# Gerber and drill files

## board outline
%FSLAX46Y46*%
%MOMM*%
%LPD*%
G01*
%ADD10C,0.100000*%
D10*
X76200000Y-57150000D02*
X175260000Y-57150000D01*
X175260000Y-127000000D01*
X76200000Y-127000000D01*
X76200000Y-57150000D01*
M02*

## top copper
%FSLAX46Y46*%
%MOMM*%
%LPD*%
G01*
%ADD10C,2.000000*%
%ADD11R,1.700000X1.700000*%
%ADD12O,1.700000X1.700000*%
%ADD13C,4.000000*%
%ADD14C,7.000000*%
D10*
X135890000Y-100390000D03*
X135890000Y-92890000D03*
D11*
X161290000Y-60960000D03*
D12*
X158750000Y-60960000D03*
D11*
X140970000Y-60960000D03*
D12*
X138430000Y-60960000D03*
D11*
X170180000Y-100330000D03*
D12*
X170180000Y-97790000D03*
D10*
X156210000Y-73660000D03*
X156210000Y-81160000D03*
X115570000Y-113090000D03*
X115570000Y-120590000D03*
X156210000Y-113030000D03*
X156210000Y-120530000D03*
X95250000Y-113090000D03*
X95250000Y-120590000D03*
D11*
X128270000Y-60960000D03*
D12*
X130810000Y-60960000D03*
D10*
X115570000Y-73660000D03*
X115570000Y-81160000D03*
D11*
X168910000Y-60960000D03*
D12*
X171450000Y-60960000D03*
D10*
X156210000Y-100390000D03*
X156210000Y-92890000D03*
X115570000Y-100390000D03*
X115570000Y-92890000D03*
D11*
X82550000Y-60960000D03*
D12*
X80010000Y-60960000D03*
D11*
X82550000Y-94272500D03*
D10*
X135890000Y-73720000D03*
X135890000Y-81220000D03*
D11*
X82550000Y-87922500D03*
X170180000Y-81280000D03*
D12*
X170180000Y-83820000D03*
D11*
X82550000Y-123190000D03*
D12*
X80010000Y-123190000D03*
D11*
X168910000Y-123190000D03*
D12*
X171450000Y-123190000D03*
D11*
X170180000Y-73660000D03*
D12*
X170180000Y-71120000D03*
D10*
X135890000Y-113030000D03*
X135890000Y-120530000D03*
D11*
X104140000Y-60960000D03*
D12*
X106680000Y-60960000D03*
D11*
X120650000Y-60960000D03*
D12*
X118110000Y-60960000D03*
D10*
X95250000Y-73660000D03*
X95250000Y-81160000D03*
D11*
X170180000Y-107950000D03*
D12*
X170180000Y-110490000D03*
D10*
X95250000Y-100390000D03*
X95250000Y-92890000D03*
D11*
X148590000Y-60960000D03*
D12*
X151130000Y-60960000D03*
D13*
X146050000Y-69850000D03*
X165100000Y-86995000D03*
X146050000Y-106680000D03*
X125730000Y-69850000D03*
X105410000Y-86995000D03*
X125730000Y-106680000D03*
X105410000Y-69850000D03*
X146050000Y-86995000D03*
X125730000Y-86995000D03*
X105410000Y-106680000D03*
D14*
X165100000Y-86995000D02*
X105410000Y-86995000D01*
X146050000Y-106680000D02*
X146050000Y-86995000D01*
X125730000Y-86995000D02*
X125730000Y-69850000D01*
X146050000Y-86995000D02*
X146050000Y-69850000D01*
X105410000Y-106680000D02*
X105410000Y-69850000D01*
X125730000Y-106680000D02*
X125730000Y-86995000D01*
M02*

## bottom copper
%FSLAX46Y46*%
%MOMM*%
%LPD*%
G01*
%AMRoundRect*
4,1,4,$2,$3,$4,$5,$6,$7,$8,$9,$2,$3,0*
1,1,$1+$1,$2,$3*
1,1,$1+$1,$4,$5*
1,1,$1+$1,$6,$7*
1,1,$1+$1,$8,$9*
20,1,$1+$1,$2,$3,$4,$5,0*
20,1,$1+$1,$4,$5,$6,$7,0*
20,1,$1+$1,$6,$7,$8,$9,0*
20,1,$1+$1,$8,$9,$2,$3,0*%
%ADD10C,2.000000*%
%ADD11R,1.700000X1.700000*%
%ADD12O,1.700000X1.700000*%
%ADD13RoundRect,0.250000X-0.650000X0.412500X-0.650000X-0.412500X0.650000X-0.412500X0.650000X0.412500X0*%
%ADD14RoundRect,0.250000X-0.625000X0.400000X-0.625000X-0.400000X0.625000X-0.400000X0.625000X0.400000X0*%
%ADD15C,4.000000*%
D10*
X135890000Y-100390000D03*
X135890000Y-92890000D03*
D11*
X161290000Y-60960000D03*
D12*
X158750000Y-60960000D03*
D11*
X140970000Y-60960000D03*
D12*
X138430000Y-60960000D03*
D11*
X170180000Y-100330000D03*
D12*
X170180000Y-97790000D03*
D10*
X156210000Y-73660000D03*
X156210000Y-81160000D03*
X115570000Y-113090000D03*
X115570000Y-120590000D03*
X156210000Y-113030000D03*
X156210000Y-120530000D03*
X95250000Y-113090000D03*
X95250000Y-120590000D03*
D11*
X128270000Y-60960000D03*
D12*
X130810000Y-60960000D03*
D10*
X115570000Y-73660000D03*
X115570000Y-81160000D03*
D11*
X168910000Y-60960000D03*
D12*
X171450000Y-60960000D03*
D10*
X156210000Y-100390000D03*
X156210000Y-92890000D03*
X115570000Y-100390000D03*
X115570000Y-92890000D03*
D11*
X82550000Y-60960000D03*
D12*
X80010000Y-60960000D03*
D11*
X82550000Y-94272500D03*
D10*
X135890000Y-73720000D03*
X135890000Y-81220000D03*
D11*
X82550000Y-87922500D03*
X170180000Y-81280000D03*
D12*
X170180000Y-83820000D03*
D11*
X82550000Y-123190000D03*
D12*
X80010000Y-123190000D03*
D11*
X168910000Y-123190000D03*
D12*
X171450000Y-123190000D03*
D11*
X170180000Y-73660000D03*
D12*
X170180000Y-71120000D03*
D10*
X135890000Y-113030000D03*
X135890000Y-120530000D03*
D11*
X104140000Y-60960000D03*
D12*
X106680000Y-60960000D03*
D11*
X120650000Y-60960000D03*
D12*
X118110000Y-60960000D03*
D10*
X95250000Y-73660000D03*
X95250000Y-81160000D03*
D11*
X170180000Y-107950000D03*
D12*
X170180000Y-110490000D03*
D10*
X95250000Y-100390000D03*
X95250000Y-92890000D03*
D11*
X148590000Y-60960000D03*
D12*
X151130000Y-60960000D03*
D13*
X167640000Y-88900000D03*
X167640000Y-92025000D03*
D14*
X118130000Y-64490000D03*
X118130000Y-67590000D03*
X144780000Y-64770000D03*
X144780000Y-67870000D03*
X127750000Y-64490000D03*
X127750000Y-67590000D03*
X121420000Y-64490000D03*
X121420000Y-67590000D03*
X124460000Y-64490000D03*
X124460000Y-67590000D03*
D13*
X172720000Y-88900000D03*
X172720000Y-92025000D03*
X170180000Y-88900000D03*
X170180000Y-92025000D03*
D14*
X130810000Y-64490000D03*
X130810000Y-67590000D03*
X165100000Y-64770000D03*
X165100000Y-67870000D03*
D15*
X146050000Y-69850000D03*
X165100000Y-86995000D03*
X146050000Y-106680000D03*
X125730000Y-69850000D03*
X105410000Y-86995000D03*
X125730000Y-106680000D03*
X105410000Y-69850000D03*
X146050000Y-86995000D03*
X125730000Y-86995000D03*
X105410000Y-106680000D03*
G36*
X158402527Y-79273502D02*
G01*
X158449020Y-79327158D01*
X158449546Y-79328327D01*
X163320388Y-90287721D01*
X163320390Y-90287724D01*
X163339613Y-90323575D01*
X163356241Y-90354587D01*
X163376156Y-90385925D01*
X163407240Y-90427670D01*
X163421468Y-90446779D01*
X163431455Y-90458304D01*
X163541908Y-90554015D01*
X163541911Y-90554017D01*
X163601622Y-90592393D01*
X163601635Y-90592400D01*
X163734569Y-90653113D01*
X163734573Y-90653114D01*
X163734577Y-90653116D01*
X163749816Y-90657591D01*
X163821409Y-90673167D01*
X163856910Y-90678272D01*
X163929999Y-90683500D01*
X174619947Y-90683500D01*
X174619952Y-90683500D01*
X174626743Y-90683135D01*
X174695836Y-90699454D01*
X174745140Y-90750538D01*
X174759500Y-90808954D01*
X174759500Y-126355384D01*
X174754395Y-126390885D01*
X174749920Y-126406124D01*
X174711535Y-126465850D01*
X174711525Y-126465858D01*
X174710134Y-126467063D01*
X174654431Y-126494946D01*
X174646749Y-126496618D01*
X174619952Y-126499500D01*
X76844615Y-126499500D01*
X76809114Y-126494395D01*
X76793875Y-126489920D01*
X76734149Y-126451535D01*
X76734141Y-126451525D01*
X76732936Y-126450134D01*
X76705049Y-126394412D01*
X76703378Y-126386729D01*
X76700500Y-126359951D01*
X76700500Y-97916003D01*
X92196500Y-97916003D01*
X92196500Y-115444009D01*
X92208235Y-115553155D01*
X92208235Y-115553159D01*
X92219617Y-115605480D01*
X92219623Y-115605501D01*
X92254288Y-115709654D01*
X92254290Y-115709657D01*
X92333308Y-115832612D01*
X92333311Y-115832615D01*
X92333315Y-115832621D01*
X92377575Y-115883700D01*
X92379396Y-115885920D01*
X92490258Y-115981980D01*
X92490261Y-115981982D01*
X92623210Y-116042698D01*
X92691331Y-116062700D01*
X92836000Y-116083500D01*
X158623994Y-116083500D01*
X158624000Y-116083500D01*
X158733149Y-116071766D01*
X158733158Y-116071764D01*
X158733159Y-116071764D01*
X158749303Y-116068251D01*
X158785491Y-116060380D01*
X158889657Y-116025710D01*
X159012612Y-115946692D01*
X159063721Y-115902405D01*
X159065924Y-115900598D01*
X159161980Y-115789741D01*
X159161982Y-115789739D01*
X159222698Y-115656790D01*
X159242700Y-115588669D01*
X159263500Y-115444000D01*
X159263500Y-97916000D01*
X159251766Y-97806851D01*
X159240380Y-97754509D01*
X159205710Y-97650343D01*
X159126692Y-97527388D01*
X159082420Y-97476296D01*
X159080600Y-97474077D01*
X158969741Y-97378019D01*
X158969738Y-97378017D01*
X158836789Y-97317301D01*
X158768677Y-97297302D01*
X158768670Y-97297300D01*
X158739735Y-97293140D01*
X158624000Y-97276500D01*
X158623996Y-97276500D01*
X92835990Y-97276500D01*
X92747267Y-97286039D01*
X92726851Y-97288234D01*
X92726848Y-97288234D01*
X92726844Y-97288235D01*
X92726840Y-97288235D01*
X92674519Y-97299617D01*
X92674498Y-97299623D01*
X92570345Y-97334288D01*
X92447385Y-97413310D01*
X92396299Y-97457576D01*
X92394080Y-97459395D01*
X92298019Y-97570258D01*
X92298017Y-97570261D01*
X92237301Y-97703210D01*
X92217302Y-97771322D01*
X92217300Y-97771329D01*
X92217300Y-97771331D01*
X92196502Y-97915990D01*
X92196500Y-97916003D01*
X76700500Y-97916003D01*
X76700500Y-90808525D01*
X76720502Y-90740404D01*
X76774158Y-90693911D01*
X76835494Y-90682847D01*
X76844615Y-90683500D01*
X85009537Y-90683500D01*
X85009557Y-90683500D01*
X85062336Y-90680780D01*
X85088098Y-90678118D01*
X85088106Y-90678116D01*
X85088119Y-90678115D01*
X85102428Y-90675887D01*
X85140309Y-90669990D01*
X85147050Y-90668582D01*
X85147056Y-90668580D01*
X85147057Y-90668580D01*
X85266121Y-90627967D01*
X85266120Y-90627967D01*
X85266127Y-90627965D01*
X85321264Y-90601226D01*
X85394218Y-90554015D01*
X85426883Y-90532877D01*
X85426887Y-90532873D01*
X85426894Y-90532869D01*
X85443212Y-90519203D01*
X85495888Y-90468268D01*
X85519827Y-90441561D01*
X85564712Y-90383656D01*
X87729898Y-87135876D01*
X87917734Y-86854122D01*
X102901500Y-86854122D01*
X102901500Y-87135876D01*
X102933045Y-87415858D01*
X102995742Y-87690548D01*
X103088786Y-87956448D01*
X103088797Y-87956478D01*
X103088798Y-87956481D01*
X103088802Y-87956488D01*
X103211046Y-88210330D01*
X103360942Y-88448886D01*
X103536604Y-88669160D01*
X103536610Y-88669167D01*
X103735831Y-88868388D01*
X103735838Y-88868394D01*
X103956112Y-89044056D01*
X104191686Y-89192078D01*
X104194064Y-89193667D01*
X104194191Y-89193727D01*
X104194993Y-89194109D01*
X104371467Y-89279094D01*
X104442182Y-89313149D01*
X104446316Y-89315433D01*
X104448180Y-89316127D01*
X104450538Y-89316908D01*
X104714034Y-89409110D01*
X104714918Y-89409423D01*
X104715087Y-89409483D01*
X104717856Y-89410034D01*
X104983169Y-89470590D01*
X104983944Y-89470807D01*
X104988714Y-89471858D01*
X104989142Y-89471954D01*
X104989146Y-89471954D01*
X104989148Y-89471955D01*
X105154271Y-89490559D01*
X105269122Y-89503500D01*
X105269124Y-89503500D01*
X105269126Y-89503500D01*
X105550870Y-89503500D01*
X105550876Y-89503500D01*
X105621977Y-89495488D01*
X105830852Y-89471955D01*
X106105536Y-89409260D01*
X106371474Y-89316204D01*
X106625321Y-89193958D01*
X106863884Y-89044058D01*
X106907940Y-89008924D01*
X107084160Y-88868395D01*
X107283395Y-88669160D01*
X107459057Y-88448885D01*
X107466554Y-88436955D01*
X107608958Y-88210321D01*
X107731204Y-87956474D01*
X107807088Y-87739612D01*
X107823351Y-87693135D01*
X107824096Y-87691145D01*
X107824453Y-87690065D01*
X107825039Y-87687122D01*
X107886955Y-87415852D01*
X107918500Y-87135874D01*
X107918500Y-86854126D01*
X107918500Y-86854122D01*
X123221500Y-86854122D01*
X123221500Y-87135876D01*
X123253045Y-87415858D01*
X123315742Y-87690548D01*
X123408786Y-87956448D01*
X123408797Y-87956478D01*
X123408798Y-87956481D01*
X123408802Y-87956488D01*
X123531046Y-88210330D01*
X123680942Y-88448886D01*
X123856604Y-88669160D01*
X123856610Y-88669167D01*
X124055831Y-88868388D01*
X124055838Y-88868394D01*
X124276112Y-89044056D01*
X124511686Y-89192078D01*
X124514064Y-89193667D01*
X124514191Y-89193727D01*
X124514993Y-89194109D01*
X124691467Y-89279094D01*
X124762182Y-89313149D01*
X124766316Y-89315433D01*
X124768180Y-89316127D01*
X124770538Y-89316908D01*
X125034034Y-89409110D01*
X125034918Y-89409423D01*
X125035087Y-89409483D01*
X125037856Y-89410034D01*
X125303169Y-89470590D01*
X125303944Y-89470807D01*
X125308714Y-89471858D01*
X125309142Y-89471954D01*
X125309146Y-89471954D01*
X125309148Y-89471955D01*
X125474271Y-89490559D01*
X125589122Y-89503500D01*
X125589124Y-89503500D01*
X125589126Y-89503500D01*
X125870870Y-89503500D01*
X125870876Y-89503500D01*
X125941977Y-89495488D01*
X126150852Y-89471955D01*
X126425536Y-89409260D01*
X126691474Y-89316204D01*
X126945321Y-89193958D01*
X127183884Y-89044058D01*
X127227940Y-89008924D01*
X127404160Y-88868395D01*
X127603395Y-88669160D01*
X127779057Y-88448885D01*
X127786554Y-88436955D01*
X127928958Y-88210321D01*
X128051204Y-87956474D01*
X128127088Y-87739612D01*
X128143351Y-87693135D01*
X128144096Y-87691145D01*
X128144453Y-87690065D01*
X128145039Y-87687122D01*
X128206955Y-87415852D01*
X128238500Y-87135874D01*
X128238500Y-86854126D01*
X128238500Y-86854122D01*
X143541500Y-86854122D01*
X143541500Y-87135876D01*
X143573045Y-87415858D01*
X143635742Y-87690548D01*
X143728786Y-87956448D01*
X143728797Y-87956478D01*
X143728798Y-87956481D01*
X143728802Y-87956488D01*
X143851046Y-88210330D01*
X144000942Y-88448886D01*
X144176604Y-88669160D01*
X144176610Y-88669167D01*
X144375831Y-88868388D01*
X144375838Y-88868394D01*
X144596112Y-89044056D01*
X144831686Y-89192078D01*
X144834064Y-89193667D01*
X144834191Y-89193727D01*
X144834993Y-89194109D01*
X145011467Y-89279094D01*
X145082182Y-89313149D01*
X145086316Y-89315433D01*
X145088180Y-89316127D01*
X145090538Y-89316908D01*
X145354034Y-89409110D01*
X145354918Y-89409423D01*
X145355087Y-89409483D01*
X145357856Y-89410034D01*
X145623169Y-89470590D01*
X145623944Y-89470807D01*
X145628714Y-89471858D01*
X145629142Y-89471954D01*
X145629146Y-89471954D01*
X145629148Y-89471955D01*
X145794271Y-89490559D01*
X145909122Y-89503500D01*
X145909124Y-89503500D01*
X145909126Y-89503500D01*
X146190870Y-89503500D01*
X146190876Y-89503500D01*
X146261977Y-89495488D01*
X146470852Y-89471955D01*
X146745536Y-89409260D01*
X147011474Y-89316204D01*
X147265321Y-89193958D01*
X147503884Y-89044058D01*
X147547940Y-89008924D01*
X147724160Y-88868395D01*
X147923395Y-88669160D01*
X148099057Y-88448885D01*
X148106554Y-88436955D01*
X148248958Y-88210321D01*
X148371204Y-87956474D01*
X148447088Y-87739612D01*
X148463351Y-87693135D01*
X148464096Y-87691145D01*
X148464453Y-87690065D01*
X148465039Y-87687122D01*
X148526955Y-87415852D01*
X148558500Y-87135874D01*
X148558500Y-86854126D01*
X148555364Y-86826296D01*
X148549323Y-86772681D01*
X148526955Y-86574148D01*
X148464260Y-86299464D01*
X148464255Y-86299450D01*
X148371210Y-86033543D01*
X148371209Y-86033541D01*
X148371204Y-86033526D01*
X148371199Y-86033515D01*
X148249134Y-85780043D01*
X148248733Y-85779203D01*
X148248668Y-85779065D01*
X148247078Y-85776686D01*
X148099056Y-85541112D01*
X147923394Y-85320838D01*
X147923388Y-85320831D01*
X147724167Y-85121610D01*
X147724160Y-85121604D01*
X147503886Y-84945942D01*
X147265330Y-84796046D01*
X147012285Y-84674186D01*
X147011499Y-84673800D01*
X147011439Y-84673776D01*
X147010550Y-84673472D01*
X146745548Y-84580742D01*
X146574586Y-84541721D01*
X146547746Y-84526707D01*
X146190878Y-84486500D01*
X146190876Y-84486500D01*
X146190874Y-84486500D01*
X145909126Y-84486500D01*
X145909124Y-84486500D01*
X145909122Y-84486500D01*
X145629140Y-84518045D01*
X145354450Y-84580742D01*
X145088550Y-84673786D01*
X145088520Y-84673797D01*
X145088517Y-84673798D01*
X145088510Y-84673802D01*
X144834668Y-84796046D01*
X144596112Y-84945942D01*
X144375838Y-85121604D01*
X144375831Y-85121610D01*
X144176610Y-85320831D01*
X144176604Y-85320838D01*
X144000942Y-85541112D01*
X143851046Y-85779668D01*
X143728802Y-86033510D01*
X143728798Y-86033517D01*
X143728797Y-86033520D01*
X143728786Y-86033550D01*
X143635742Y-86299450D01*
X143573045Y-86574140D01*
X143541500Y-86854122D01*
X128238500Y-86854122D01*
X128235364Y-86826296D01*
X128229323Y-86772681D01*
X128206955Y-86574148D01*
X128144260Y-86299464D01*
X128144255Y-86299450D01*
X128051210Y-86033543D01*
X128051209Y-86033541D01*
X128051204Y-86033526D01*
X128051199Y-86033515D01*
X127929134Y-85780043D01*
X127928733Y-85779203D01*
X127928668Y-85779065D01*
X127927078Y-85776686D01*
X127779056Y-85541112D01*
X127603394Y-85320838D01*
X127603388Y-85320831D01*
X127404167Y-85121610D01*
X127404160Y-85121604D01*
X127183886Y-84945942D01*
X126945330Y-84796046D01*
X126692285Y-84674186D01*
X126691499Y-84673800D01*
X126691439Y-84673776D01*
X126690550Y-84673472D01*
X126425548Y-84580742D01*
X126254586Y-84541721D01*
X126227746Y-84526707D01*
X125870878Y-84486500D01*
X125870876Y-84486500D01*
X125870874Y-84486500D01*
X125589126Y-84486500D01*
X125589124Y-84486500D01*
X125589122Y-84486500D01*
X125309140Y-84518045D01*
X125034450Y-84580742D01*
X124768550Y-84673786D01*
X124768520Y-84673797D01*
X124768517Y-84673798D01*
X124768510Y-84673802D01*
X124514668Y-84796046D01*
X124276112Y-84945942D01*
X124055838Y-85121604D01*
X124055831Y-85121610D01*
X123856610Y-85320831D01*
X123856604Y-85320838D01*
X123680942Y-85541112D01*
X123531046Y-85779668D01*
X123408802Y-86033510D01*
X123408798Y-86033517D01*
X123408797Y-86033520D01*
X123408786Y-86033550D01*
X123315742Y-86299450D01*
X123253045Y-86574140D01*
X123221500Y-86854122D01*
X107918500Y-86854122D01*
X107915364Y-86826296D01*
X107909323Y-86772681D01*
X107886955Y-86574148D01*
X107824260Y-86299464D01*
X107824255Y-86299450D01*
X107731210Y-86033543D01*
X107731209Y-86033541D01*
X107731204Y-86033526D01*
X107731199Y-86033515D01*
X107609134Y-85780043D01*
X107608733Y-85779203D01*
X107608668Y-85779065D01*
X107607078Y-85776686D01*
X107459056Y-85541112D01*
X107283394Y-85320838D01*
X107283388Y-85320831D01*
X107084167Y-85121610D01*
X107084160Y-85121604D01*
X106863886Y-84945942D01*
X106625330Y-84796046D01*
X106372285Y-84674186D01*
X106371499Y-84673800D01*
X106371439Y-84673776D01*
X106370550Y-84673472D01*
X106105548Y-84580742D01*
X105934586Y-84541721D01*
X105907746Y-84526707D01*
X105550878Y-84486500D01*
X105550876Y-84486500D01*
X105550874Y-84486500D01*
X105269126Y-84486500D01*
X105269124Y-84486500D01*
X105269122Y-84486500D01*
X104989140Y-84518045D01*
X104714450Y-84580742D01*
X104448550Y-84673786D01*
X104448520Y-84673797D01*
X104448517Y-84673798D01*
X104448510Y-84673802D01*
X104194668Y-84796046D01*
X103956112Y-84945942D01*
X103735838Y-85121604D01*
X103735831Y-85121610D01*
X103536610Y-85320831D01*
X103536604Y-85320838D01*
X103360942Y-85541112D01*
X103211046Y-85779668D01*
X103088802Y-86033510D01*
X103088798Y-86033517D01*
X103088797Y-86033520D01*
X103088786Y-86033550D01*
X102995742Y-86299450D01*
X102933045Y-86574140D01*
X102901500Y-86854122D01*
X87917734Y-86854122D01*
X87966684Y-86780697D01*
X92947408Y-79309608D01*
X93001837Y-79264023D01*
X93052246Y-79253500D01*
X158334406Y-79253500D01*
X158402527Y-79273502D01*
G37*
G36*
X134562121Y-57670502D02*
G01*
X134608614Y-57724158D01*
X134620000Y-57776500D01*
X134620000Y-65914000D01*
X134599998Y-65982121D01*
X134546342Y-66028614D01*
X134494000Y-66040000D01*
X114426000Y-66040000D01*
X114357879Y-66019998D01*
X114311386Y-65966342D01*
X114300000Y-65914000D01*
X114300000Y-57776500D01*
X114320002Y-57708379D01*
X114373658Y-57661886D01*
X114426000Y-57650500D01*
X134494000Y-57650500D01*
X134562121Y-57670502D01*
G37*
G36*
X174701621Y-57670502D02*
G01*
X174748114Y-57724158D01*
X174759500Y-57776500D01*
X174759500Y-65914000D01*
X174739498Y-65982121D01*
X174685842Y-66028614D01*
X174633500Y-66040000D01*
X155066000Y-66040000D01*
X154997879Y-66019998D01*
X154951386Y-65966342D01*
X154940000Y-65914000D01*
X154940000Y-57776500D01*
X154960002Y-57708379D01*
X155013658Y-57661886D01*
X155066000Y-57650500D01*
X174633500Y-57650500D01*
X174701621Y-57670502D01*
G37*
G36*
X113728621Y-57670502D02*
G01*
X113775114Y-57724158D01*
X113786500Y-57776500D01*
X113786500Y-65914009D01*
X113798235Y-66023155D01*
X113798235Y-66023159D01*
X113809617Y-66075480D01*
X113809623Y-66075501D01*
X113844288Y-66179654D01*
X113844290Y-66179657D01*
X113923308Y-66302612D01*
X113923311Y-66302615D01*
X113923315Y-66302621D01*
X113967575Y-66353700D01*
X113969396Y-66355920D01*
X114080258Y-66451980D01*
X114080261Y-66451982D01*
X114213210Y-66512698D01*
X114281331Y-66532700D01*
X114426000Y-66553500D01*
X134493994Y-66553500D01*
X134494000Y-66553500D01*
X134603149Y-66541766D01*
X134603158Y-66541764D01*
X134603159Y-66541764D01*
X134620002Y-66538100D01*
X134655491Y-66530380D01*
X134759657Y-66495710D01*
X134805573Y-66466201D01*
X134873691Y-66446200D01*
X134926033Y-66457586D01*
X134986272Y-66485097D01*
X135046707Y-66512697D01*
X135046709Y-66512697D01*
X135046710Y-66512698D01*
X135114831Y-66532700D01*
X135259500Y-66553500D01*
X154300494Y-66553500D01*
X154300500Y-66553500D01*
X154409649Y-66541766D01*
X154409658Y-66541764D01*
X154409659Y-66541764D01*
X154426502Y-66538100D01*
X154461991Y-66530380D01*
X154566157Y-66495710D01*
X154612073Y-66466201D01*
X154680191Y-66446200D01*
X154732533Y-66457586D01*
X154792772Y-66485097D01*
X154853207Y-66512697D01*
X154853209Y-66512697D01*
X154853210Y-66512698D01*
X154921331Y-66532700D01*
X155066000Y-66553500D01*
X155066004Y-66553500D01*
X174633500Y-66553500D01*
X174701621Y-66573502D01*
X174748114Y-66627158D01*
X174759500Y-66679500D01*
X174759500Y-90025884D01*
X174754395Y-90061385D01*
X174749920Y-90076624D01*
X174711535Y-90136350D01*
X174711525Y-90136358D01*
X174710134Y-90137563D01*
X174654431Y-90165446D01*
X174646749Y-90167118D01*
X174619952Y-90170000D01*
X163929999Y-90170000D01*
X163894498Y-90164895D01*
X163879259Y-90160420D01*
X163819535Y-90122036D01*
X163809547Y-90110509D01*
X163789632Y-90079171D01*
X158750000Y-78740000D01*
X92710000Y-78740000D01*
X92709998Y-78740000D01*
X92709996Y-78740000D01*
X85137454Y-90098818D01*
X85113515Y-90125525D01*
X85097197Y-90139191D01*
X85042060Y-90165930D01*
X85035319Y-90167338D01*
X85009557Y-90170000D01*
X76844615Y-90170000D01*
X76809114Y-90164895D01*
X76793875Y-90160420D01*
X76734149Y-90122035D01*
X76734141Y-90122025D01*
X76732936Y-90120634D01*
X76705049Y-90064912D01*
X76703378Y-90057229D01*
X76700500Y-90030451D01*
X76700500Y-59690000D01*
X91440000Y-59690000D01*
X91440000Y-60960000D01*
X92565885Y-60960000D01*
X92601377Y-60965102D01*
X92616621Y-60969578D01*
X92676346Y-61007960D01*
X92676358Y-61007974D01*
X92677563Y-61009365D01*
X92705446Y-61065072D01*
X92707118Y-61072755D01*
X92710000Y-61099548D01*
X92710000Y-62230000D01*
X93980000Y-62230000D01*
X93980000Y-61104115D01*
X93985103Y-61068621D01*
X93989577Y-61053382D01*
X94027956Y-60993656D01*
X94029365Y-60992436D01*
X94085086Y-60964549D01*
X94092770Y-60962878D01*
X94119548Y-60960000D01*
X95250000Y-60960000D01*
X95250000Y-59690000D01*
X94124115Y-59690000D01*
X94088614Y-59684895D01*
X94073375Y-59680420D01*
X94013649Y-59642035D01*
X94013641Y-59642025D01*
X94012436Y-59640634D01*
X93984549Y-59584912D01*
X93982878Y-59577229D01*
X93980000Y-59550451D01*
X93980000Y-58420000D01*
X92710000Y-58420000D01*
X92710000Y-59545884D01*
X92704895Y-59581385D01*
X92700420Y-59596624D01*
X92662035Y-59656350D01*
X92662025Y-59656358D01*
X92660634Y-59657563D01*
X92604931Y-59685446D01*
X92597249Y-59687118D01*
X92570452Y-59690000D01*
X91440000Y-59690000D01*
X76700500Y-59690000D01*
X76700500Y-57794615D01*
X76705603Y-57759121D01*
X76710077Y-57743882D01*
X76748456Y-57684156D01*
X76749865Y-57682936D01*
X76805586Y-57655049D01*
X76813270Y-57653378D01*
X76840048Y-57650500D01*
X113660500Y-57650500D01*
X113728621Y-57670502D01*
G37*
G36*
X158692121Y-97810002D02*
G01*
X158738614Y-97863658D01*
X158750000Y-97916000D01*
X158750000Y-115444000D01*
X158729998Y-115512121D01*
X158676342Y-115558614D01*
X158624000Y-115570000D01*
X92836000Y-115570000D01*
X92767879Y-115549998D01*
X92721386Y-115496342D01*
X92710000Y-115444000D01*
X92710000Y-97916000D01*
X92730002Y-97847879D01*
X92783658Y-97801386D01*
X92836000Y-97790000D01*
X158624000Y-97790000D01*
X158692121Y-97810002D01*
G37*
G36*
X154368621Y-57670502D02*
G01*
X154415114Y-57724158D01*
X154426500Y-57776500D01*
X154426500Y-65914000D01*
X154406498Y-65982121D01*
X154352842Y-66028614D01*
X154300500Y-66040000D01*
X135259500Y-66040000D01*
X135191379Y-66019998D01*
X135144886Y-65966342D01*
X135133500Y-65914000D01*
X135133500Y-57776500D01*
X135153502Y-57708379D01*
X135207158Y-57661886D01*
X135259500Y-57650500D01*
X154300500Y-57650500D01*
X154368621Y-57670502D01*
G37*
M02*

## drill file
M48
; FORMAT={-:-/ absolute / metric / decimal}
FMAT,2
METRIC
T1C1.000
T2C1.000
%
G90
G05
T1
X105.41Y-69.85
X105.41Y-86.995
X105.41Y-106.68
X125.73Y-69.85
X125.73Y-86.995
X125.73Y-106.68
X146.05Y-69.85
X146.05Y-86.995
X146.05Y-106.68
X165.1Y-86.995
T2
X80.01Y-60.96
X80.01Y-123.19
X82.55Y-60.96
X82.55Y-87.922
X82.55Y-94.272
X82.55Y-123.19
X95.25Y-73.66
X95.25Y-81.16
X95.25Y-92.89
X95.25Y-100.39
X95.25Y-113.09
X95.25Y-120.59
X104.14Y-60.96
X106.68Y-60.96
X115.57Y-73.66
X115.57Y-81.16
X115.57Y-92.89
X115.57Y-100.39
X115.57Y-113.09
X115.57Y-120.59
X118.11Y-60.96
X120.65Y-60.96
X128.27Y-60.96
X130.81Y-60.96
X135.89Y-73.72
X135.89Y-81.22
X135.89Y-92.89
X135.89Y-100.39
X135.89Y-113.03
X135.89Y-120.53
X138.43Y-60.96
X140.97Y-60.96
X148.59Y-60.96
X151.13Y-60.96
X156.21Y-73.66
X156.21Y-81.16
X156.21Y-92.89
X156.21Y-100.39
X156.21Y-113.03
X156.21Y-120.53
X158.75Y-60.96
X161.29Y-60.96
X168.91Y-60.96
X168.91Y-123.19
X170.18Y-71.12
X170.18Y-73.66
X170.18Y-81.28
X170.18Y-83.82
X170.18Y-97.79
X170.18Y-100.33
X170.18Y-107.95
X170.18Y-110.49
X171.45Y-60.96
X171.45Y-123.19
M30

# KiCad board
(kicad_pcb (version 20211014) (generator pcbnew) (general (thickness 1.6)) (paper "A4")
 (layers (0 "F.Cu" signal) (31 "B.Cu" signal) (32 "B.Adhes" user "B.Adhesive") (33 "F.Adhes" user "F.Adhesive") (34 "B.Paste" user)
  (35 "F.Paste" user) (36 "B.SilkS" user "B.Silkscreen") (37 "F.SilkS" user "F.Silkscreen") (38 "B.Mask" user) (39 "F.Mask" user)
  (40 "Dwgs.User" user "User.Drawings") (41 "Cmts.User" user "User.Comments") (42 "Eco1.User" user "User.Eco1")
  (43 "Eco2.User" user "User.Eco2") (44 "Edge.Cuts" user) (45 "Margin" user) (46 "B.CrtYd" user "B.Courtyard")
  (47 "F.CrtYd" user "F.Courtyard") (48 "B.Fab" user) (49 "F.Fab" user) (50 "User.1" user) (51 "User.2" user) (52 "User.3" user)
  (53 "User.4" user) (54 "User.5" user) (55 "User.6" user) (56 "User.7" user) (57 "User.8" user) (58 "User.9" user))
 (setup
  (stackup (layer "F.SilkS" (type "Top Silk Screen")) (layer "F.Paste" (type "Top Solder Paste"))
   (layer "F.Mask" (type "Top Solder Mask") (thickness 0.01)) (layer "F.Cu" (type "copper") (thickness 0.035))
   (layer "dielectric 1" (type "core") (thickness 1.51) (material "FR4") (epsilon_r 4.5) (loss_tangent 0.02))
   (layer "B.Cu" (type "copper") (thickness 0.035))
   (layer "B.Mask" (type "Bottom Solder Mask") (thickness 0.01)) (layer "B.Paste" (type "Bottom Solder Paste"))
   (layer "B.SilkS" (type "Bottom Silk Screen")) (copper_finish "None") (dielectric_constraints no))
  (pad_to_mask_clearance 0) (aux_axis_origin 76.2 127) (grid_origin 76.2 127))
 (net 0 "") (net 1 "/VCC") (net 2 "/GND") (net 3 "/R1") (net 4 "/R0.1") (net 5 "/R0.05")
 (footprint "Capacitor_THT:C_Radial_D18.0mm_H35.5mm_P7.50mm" (layer "F.Cu") (at 135.89 100.39 90)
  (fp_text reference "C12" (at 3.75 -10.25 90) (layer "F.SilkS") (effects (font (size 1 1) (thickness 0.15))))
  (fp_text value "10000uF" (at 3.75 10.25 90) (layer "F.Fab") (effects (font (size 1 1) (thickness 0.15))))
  (pad "1" thru_hole circle (at 0 0 90) (size 2 2) (drill 1) (layers *.Cu *.Mask) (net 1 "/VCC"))
  (pad "2" thru_hole circle (at 7.5 0 90) (size 2 2) (drill 1) (layers *.Cu *.Mask) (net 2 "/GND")))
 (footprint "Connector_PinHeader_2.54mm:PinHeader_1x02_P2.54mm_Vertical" (layer "F.Cu") (at 161.29 60.96 -90)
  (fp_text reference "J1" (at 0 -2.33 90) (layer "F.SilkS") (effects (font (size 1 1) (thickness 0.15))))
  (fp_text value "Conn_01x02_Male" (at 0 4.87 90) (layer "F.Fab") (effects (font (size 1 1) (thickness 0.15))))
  (pad "1" thru_hole rect (at 0 0 270) (size 1.7 1.7) (drill 1) (layers *.Cu *.Mask) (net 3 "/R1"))
  (pad "2" thru_hole oval (at 0 2.54 270) (size 1.7 1.7) (drill 1) (layers *.Cu *.Mask) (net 3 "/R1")))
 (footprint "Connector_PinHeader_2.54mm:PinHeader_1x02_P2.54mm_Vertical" (layer "F.Cu") (at 140.97 60.96 -90)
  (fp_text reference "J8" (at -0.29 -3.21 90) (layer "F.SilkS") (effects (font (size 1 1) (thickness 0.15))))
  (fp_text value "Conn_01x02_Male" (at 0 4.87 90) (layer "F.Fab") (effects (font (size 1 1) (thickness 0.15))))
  (pad "1" thru_hole rect (at 0 0 270) (size 1.7 1.7) (drill 1) (layers *.Cu *.Mask) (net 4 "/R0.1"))
  (pad "2" thru_hole oval (at 0 2.54 270) (size 1.7 1.7) (drill 1) (layers *.Cu *.Mask) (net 4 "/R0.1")))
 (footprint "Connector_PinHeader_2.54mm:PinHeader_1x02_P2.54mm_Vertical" (layer "F.Cu") (at 170.18 100.33 180)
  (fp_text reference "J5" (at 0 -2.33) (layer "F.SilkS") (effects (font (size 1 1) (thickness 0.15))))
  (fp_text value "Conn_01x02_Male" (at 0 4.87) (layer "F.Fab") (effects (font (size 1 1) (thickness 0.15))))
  (pad "1" thru_hole rect (at 0 0 180) (size 1.7 1.7) (drill 1) (layers *.Cu *.Mask) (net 2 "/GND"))
  (pad "2" thru_hole oval (at 0 2.54 180) (size 1.7 1.7) (drill 1) (layers *.Cu *.Mask) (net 2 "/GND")))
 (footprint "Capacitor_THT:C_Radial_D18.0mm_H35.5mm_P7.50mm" (layer "F.Cu") (at 156.21 73.66 -90)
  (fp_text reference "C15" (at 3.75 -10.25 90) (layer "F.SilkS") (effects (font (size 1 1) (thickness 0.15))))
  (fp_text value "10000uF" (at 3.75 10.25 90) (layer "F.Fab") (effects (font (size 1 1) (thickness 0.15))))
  (pad "1" thru_hole circle (at 0 0 270) (size 2 2) (drill 1) (layers *.Cu *.Mask) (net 1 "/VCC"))
  (pad "2" thru_hole circle (at 7.5 0 270) (size 2 2) (drill 1) (layers *.Cu *.Mask) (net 2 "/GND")))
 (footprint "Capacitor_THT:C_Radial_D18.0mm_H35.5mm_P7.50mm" (layer "F.Cu") (at 115.57 113.09 -90)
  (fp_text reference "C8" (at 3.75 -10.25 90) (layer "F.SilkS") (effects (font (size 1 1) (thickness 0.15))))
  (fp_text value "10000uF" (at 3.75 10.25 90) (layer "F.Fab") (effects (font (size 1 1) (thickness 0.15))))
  (pad "1" thru_hole circle (at 0 0 270) (size 2 2) (drill 1) (layers *.Cu *.Mask) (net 1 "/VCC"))
  (pad "2" thru_hole circle (at 7.5 0 270) (size 2 2) (drill 1) (layers *.Cu *.Mask) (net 2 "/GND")))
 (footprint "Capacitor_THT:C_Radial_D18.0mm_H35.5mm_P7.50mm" (layer "F.Cu") (at 156.21 113.03 -90)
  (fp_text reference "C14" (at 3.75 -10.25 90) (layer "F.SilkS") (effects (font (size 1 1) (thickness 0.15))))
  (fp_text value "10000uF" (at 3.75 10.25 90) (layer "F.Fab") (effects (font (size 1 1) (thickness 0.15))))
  (pad "1" thru_hole circle (at 0 0 270) (size 2 2) (drill 1) (layers *.Cu *.Mask) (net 1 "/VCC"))
  (pad "2" thru_hole circle (at 7.5 0 270) (size 2 2) (drill 1) (layers *.Cu *.Mask) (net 2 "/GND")))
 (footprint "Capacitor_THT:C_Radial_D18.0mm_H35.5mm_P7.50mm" (layer "F.Cu") (at 95.25 113.09 -90)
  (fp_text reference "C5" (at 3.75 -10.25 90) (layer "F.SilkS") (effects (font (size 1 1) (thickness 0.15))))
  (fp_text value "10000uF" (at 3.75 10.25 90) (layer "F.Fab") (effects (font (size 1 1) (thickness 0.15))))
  (pad "1" thru_hole circle (at 0 0 270) (size 2 2) (drill 1) (layers *.Cu *.Mask) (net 1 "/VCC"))
  (pad "2" thru_hole circle (at 7.5 0 270) (size 2 2) (drill 1) (layers *.Cu *.Mask) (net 2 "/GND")))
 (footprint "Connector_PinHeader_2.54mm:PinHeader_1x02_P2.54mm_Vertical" (layer "F.Cu") (at 128.27 60.96 90)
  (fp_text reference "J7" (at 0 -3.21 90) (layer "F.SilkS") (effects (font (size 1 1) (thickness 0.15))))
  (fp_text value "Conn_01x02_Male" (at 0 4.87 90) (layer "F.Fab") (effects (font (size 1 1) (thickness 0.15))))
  (pad "1" thru_hole rect (at 0 0 90) (size 1.7 1.7) (drill 1) (layers *.Cu *.Mask) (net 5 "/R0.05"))
  (pad "2" thru_hole oval (at 0 2.54 90) (size 1.7 1.7) (drill 1) (layers *.Cu *.Mask) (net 5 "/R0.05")))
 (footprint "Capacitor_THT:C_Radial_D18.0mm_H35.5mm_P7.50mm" (layer "F.Cu") (at 115.57 73.66 -90)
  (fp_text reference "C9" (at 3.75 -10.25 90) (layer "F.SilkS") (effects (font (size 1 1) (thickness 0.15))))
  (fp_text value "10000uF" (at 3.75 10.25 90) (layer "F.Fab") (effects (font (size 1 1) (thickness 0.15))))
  (pad "1" thru_hole circle (at 0 0 270) (size 2 2) (drill 1) (layers *.Cu *.Mask) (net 1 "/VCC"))
  (pad "2" thru_hole circle (at 7.5 0 270) (size 2 2) (drill 1) (layers *.Cu *.Mask) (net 2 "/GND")))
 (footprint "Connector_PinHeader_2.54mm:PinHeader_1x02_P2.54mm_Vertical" (layer "F.Cu") (at 168.91 60.96 90)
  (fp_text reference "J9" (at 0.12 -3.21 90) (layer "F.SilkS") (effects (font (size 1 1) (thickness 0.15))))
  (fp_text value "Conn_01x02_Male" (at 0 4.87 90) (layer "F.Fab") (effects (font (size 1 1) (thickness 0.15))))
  (pad "1" thru_hole rect (at 0 0 90) (size 1.7 1.7) (drill 1) (layers *.Cu *.Mask) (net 3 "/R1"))
  (pad "2" thru_hole oval (at 0 2.54 90) (size 1.7 1.7) (drill 1) (layers *.Cu *.Mask) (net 3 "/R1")))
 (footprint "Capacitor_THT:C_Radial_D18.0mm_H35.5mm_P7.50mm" (layer "F.Cu") (at 156.21 100.39 90)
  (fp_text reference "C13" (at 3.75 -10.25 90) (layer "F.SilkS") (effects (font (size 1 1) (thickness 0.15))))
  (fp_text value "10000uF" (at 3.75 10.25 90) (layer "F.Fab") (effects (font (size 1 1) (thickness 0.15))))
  (pad "1" thru_hole circle (at 0 0 90) (size 2 2) (drill 1) (layers *.Cu *.Mask) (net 1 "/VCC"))
  (pad "2" thru_hole circle (at 7.5 0 90) (size 2 2) (drill 1) (layers *.Cu *.Mask) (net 2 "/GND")))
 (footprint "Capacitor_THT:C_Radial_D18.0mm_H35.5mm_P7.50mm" (layer "F.Cu") (at 115.57 100.39 90)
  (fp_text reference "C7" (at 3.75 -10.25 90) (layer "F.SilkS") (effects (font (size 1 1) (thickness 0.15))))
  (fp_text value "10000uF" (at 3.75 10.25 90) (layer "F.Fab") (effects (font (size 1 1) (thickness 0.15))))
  (pad "1" thru_hole circle (at 0 0 90) (size 2 2) (drill 1) (layers *.Cu *.Mask) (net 1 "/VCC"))
  (pad "2" thru_hole circle (at 7.5 0 90) (size 2 2) (drill 1) (layers *.Cu *.Mask) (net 2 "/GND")))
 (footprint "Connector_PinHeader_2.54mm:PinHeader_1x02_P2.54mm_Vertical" (layer "F.Cu") (at 82.55 60.96 -90)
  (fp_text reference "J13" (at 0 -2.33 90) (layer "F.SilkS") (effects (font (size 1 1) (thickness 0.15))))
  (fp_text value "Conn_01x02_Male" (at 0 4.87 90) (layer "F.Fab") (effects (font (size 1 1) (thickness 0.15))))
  (pad "1" thru_hole rect (at 0 0 270) (size 1.7 1.7) (drill 1) (layers *.Cu *.Mask) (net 1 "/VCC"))
  (pad "2" thru_hole oval (at 0 2.54 270) (size 1.7 1.7) (drill 1) (layers *.Cu *.Mask) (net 1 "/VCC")))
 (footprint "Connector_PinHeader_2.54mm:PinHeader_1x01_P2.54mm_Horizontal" (layer "F.Cu") (at 82.55 94.2725 180)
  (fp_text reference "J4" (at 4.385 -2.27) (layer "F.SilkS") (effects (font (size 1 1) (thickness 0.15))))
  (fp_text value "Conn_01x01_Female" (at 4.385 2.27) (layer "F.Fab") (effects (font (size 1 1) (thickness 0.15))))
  (pad "1" thru_hole rect (at 0 0 180) (size 1.7 1.7) (drill 1) (layers *.Cu *.Mask) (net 2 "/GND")))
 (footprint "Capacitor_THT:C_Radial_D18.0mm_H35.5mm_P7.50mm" (layer "F.Cu") (at 135.89 73.72 -90)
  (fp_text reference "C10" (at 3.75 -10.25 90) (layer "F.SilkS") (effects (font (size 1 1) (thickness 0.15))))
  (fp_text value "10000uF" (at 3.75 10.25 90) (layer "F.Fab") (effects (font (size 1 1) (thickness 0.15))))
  (pad "1" thru_hole circle (at 0 0 270) (size 2 2) (drill 1) (layers *.Cu *.Mask) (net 1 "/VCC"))
  (pad "2" thru_hole circle (at 7.5 0 270) (size 2 2) (drill 1) (layers *.Cu *.Mask) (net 2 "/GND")))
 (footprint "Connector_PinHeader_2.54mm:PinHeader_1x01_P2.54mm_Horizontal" (layer "F.Cu") (at 82.55 87.9225 180)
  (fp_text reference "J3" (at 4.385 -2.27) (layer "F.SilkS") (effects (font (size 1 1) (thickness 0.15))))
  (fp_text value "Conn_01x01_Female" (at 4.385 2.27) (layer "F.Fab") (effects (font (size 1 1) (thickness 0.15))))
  (pad "1" thru_hole rect (at 0 0 180) (size 1.7 1.7) (drill 1) (layers *.Cu *.Mask) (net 1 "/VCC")))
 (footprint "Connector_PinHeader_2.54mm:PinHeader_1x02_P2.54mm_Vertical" (layer "F.Cu") (at 170.18 81.28)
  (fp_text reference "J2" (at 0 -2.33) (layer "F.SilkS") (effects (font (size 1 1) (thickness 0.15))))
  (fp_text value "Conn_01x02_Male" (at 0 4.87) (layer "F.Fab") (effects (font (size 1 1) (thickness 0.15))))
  (pad "1" thru_hole rect (at 0 0) (size 1.7 1.7) (drill 1) (layers *.Cu *.Mask) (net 1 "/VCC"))
  (pad "2" thru_hole oval (at 0 2.54) (size 1.7 1.7) (drill 1) (layers *.Cu *.Mask) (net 1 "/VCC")))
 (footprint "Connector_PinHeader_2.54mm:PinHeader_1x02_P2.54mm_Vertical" (layer "F.Cu") (at 82.55 123.19 -90)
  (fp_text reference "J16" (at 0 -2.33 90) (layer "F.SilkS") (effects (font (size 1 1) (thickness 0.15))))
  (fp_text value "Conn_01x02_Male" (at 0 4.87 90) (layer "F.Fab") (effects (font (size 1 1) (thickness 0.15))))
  (pad "1" thru_hole rect (at 0 0 270) (size 1.7 1.7) (drill 1) (layers *.Cu *.Mask) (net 2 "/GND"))
  (pad "2" thru_hole oval (at 0 2.54 270) (size 1.7 1.7) (drill 1) (layers *.Cu *.Mask) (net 2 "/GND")))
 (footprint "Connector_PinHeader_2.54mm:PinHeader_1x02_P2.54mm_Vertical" (layer "F.Cu") (at 168.91 123.19 90)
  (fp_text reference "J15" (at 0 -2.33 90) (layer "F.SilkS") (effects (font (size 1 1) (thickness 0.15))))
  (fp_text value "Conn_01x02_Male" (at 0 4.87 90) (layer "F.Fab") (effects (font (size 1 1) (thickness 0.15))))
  (pad "1" thru_hole rect (at 0 0 90) (size 1.7 1.7) (drill 1) (layers *.Cu *.Mask) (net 2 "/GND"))
  (pad "2" thru_hole oval (at 0 2.54 90) (size 1.7 1.7) (drill 1) (layers *.Cu *.Mask) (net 2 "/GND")))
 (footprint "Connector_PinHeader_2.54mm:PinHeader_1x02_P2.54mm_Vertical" (layer "F.Cu") (at 170.18 73.66 180)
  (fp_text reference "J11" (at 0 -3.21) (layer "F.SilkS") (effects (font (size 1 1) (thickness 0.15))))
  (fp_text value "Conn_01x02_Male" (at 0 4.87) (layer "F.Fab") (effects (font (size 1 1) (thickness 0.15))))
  (pad "1" thru_hole rect (at 0 0 180) (size 1.7 1.7) (drill 1) (layers *.Cu *.Mask) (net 1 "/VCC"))
  (pad "2" thru_hole oval (at 0 2.54 180) (size 1.7 1.7) (drill 1) (layers *.Cu *.Mask) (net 1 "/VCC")))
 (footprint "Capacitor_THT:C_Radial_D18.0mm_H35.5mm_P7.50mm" (layer "F.Cu") (at 135.89 113.03 -90)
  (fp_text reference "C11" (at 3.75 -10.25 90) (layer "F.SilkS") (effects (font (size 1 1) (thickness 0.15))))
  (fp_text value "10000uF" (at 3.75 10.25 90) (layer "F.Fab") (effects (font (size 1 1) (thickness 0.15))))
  (pad "1" thru_hole circle (at 0 0 270) (size 2 2) (drill 1) (layers *.Cu *.Mask) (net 1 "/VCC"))
  (pad "2" thru_hole circle (at 7.5 0 270) (size 2 2) (drill 1) (layers *.Cu *.Mask) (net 2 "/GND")))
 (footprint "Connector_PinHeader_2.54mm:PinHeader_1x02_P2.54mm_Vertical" (layer "F.Cu") (at 104.14 60.96 90)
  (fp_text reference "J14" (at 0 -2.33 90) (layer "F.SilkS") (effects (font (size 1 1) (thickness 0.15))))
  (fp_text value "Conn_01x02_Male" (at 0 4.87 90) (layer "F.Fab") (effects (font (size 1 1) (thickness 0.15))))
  (pad "1" thru_hole rect (at 0 0 90) (size 1.7 1.7) (drill 1) (layers *.Cu *.Mask) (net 1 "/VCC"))
  (pad "2" thru_hole oval (at 0 2.54 90) (size 1.7 1.7) (drill 1) (layers *.Cu *.Mask) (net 1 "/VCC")))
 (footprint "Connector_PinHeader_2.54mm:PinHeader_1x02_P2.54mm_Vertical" (layer "F.Cu") (at 120.65 60.96 -90)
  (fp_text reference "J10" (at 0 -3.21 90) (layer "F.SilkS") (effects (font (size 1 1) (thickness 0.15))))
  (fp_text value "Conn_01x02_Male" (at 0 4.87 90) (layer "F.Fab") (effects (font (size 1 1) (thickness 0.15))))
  (pad "1" thru_hole rect (at 0 0 270) (size 1.7 1.7) (drill 1) (layers *.Cu *.Mask) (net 5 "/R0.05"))
  (pad "2" thru_hole oval (at 0 2.54 270) (size 1.7 1.7) (drill 1) (layers *.Cu *.Mask) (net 5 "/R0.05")))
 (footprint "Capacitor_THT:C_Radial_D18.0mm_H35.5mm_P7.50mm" (layer "F.Cu") (at 95.25 73.66 -90)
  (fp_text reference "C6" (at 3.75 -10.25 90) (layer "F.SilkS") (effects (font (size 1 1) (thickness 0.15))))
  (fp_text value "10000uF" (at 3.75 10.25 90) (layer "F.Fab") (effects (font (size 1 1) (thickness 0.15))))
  (pad "1" thru_hole circle (at 0 0 270) (size 2 2) (drill 1) (layers *.Cu *.Mask) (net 1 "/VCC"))
  (pad "2" thru_hole circle (at 7.5 0 270) (size 2 2) (drill 1) (layers *.Cu *.Mask) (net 2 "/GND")))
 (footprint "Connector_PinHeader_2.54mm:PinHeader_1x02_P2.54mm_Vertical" (layer "F.Cu") (at 170.18 107.95)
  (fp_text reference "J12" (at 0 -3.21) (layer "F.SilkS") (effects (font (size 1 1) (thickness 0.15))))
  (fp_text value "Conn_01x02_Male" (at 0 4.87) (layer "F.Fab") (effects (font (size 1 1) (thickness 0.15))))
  (pad "1" thru_hole rect (at 0 0) (size 1.7 1.7) (drill 1) (layers *.Cu *.Mask) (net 2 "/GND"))
  (pad "2" thru_hole oval (at 0 2.54) (size 1.7 1.7) (drill 1) (layers *.Cu *.Mask) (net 2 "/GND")))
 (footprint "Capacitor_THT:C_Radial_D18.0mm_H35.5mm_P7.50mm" (layer "F.Cu") (at 95.25 100.39 90)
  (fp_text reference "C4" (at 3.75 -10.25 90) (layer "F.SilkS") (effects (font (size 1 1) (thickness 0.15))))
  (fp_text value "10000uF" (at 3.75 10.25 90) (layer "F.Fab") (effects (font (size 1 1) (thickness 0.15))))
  (pad "1" thru_hole circle (at 0 0 90) (size 2 2) (drill 1) (layers *.Cu *.Mask) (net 1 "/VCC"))
  (pad "2" thru_hole circle (at 7.5 0 90) (size 2 2) (drill 1) (layers *.Cu *.Mask) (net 2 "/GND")))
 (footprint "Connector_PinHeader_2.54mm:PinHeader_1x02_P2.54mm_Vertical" (layer "F.Cu") (at 148.59 60.96 90)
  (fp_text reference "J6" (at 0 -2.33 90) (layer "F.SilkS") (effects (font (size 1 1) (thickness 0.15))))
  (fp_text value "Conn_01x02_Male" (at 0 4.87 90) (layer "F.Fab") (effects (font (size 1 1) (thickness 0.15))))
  (pad "1" thru_hole rect (at 0 0 90) (size 1.7 1.7) (drill 1) (layers *.Cu *.Mask) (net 4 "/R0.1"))
  (pad "2" thru_hole oval (at 0 2.54 90) (size 1.7 1.7) (drill 1) (layers *.Cu *.Mask) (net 4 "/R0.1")))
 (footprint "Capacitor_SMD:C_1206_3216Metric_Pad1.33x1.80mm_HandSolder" (layer "B.Cu") (at 167.64 90.4625 -90)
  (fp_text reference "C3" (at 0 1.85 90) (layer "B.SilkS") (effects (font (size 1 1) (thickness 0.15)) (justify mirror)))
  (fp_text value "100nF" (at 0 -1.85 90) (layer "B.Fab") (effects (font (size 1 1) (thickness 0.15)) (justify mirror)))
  (pad "1" smd roundrect (at -1.5625 0 270) (size 1.325 1.8) (layers "B.Cu" "B.Paste" "B.Mask") (roundrect_rratio 0.1886792453)
   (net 1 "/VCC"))
  (pad "2" smd roundrect (at 1.5625 0 270) (size 1.325 1.8) (layers "B.Cu" "B.Paste" "B.Mask") (roundrect_rratio 0.1886792453)
   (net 2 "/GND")))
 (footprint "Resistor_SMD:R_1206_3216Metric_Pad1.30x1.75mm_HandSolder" (layer "B.Cu") (at 118.13 66.04 -90)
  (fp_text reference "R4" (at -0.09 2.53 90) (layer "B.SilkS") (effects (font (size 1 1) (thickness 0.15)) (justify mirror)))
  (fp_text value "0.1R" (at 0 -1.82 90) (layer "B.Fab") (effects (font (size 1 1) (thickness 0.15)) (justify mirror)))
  (pad "1" smd roundrect (at -1.55 0 270) (size 1.3 1.75) (layers "B.Cu" "B.Paste" "B.Mask") (roundrect_rratio 0.192308) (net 5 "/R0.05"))
  (pad "2" smd roundrect (at 1.55 0 270) (size 1.3 1.75) (layers "B.Cu" "B.Paste" "B.Mask") (roundrect_rratio 0.192308) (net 1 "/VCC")))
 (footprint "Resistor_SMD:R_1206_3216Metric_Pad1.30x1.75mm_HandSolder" (layer "B.Cu") (at 144.78 66.32 -90)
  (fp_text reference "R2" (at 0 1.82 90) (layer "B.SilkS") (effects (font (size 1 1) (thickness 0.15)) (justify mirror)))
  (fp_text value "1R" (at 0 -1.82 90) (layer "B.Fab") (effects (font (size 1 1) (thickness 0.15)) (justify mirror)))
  (pad "1" smd roundrect (at -1.55 0 270) (size 1.3 1.75) (layers "B.Cu" "B.Paste" "B.Mask") (roundrect_rratio 0.1923076923) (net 4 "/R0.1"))
  (pad "2" smd roundrect (at 1.55 0 270) (size 1.3 1.75) (layers "B.Cu" "B.Paste" "B.Mask") (roundrect_rratio 0.1923076923) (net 1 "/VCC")))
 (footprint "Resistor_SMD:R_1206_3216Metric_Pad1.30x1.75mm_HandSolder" (layer "B.Cu") (at 127.75 66.04 -90)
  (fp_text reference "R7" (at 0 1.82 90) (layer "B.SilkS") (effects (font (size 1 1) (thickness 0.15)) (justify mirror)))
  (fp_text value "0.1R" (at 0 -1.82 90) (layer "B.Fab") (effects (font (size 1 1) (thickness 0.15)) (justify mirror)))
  (pad "1" smd roundrect (at -1.55 0 270) (size 1.3 1.75) (layers "B.Cu" "B.Paste" "B.Mask") (roundrect_rratio 0.192308) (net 5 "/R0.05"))
  (pad "2" smd roundrect (at 1.55 0 270) (size 1.3 1.75) (layers "B.Cu" "B.Paste" "B.Mask") (roundrect_rratio 0.192308) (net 1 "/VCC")))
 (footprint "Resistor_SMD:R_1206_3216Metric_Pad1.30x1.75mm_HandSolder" (layer "B.Cu") (at 121.42 66.04 -90)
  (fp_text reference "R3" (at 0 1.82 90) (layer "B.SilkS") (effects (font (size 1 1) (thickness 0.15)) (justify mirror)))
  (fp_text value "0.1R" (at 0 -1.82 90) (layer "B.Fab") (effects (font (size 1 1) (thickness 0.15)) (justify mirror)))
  (pad "1" smd roundrect (at -1.55 0 270) (size 1.3 1.75) (layers "B.Cu" "B.Paste" "B.Mask") (roundrect_rratio 0.192308) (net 5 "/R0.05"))
  (pad "2" smd roundrect (at 1.55 0 270) (size 1.3 1.75) (layers "B.Cu" "B.Paste" "B.Mask") (roundrect_rratio 0.192308) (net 1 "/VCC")))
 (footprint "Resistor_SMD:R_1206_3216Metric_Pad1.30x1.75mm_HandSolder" (layer "B.Cu") (at 124.46 66.04 -90)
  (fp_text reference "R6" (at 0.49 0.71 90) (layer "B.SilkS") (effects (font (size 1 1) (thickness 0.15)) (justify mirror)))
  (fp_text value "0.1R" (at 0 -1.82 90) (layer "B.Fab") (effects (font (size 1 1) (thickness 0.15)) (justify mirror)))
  (pad "1" smd roundrect (at -1.55 0 270) (size 1.3 1.75) (layers "B.Cu" "B.Paste" "B.Mask") (roundrect_rratio 0.192308) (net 5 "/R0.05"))
  (pad "2" smd roundrect (at 1.55 0 270) (size 1.3 1.75) (layers "B.Cu" "B.Paste" "B.Mask") (roundrect_rratio 0.192308) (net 1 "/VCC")))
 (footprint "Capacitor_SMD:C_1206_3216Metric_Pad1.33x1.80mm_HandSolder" (layer "B.Cu") (at 172.72 90.4625 -90)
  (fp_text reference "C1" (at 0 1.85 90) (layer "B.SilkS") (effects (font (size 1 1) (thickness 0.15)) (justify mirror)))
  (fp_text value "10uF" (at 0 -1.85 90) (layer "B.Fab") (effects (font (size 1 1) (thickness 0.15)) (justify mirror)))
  (pad "1" smd roundrect (at -1.5625 0 270) (size 1.325 1.8) (layers "B.Cu" "B.Paste" "B.Mask") (roundrect_rratio 0.1886792453)
   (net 1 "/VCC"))
  (pad "2" smd roundrect (at 1.5625 0 270) (size 1.325 1.8) (layers "B.Cu" "B.Paste" "B.Mask") (roundrect_rratio 0.1886792453)
   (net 2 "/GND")))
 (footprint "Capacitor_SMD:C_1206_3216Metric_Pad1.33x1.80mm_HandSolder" (layer "B.Cu") (at 170.18 90.4625 -90)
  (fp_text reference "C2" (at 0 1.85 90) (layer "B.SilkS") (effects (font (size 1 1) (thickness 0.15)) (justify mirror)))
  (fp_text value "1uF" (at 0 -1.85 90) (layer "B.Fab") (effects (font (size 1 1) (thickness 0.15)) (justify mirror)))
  (pad "1" smd roundrect (at -1.5625 0 270) (size 1.325 1.8) (layers "B.Cu" "B.Paste" "B.Mask") (roundrect_rratio 0.1886792453)
   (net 1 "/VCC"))
  (pad "2" smd roundrect (at 1.5625 0 270) (size 1.325 1.8) (layers "B.Cu" "B.Paste" "B.Mask") (roundrect_rratio 0.1886792453)
   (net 2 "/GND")))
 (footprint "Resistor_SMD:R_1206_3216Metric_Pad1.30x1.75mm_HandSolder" (layer "B.Cu") (at 130.81 66.04 -90)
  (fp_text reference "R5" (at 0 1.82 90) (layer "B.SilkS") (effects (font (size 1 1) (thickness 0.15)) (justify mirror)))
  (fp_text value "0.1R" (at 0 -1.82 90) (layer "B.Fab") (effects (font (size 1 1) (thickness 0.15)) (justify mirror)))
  (pad "1" smd roundrect (at -1.55 0 270) (size 1.3 1.75) (layers "B.Cu" "B.Paste" "B.Mask") (roundrect_rratio 0.192308) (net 5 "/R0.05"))
  (pad "2" smd roundrect (at 1.55 0 270) (size 1.3 1.75) (layers "B.Cu" "B.Paste" "B.Mask") (roundrect_rratio 0.192308) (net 1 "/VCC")))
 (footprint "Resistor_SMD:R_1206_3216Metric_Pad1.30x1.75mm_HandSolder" (layer "B.Cu") (at 165.1 66.32 -90)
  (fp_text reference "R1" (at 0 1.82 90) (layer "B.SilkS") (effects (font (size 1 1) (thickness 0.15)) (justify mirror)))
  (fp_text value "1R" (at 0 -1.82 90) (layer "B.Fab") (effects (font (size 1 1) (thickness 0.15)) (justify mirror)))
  (pad "1" smd roundrect (at -1.55 0 270) (size 1.3 1.75) (layers "B.Cu" "B.Paste" "B.Mask") (roundrect_rratio 0.1923076923) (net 3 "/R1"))
  (pad "2" smd roundrect (at 1.55 0 270) (size 1.3 1.75) (layers "B.Cu" "B.Paste" "B.Mask") (roundrect_rratio 0.1923076923) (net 1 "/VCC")))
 (gr_rect (start 76.2 127) (end 175.26 57.15) (layer "Edge.Cuts") (width 0.1) (fill none))
 (segment (start 165.1 86.995) (end 105.41 86.995) (width 7) (layer "F.Cu") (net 1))
 (segment (start 146.05 106.68) (end 146.05 86.995) (width 7) (layer "F.Cu") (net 1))
 (segment (start 125.73 86.995) (end 125.73 69.85) (width 7) (layer "F.Cu") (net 1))
 (segment (start 146.05 86.995) (end 146.05 69.85) (width 7) (layer "F.Cu") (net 1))
 (segment (start 105.41 106.68) (end 105.41 69.85) (width 7) (layer "F.Cu") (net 1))
 (segment (start 125.73 106.68) (end 125.73 86.995) (width 7) (layer "F.Cu") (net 1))
 (via (at 146.05 69.85) (size 4) (drill 1) (layers "F.Cu" "B.Cu") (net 1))
 (via (at 165.1 86.995) (size 4) (drill 1) (layers "F.Cu" "B.Cu") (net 1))
 (via (at 146.05 106.68) (size 4) (drill 1) (layers "F.Cu" "B.Cu") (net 1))
 (via (at 125.73 69.85) (size 4) (drill 1) (layers "F.Cu" "B.Cu") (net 1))
 (via (at 105.41 86.995) (size 4) (drill 1) (layers "F.Cu" "B.Cu") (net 1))
 (via (at 125.73 106.68) (size 4) (drill 1) (layers "F.Cu" "B.Cu") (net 1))
 (via (at 105.41 69.85) (size 4) (drill 1) (layers "F.Cu" "B.Cu") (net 1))
 (via (at 146.05 86.995) (size 4) (drill 1) (layers "F.Cu" "B.Cu") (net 1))
 (via (at 125.73 86.995) (size 4) (drill 1) (layers "F.Cu" "B.Cu") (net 1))
 (via (at 105.41 106.68) (size 4) (drill 1) (layers "F.Cu" "B.Cu") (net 1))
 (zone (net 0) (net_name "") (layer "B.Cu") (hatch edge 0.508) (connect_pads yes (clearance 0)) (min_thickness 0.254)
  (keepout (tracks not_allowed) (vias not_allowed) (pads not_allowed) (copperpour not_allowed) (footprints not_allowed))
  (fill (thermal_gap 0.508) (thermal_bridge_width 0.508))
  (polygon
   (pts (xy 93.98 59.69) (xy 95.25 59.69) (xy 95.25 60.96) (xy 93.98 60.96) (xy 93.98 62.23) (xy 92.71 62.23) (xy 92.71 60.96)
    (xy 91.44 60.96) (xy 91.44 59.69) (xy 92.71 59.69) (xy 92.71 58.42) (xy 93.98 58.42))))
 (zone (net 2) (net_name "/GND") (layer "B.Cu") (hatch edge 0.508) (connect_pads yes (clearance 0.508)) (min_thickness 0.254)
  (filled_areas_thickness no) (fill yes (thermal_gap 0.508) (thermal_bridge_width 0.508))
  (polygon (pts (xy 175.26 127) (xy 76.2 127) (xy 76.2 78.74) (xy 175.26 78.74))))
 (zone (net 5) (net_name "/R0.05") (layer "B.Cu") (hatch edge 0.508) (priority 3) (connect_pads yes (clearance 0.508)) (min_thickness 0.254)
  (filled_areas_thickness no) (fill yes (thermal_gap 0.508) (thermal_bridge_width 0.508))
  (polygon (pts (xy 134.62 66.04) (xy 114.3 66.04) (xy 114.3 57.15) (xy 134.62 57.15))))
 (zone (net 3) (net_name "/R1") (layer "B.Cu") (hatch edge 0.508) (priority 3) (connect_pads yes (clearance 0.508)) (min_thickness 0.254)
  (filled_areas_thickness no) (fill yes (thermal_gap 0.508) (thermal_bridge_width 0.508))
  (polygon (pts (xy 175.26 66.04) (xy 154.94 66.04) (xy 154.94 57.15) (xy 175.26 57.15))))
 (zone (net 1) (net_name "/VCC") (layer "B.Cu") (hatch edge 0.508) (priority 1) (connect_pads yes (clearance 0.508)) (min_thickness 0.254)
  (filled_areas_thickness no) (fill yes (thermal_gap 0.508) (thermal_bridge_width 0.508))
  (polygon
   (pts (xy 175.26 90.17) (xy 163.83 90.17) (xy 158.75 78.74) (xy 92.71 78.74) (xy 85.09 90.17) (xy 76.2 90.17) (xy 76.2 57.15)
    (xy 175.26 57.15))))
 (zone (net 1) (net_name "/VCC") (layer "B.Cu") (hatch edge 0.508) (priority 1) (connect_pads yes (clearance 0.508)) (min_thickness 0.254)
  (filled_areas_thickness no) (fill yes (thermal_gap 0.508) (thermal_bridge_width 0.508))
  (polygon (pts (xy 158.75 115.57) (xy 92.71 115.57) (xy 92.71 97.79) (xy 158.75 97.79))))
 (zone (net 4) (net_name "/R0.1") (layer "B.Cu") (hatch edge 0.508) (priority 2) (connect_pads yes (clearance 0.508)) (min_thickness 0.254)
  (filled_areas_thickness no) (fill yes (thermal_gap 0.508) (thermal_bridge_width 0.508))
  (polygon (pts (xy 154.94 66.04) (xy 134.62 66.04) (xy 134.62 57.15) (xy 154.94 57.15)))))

